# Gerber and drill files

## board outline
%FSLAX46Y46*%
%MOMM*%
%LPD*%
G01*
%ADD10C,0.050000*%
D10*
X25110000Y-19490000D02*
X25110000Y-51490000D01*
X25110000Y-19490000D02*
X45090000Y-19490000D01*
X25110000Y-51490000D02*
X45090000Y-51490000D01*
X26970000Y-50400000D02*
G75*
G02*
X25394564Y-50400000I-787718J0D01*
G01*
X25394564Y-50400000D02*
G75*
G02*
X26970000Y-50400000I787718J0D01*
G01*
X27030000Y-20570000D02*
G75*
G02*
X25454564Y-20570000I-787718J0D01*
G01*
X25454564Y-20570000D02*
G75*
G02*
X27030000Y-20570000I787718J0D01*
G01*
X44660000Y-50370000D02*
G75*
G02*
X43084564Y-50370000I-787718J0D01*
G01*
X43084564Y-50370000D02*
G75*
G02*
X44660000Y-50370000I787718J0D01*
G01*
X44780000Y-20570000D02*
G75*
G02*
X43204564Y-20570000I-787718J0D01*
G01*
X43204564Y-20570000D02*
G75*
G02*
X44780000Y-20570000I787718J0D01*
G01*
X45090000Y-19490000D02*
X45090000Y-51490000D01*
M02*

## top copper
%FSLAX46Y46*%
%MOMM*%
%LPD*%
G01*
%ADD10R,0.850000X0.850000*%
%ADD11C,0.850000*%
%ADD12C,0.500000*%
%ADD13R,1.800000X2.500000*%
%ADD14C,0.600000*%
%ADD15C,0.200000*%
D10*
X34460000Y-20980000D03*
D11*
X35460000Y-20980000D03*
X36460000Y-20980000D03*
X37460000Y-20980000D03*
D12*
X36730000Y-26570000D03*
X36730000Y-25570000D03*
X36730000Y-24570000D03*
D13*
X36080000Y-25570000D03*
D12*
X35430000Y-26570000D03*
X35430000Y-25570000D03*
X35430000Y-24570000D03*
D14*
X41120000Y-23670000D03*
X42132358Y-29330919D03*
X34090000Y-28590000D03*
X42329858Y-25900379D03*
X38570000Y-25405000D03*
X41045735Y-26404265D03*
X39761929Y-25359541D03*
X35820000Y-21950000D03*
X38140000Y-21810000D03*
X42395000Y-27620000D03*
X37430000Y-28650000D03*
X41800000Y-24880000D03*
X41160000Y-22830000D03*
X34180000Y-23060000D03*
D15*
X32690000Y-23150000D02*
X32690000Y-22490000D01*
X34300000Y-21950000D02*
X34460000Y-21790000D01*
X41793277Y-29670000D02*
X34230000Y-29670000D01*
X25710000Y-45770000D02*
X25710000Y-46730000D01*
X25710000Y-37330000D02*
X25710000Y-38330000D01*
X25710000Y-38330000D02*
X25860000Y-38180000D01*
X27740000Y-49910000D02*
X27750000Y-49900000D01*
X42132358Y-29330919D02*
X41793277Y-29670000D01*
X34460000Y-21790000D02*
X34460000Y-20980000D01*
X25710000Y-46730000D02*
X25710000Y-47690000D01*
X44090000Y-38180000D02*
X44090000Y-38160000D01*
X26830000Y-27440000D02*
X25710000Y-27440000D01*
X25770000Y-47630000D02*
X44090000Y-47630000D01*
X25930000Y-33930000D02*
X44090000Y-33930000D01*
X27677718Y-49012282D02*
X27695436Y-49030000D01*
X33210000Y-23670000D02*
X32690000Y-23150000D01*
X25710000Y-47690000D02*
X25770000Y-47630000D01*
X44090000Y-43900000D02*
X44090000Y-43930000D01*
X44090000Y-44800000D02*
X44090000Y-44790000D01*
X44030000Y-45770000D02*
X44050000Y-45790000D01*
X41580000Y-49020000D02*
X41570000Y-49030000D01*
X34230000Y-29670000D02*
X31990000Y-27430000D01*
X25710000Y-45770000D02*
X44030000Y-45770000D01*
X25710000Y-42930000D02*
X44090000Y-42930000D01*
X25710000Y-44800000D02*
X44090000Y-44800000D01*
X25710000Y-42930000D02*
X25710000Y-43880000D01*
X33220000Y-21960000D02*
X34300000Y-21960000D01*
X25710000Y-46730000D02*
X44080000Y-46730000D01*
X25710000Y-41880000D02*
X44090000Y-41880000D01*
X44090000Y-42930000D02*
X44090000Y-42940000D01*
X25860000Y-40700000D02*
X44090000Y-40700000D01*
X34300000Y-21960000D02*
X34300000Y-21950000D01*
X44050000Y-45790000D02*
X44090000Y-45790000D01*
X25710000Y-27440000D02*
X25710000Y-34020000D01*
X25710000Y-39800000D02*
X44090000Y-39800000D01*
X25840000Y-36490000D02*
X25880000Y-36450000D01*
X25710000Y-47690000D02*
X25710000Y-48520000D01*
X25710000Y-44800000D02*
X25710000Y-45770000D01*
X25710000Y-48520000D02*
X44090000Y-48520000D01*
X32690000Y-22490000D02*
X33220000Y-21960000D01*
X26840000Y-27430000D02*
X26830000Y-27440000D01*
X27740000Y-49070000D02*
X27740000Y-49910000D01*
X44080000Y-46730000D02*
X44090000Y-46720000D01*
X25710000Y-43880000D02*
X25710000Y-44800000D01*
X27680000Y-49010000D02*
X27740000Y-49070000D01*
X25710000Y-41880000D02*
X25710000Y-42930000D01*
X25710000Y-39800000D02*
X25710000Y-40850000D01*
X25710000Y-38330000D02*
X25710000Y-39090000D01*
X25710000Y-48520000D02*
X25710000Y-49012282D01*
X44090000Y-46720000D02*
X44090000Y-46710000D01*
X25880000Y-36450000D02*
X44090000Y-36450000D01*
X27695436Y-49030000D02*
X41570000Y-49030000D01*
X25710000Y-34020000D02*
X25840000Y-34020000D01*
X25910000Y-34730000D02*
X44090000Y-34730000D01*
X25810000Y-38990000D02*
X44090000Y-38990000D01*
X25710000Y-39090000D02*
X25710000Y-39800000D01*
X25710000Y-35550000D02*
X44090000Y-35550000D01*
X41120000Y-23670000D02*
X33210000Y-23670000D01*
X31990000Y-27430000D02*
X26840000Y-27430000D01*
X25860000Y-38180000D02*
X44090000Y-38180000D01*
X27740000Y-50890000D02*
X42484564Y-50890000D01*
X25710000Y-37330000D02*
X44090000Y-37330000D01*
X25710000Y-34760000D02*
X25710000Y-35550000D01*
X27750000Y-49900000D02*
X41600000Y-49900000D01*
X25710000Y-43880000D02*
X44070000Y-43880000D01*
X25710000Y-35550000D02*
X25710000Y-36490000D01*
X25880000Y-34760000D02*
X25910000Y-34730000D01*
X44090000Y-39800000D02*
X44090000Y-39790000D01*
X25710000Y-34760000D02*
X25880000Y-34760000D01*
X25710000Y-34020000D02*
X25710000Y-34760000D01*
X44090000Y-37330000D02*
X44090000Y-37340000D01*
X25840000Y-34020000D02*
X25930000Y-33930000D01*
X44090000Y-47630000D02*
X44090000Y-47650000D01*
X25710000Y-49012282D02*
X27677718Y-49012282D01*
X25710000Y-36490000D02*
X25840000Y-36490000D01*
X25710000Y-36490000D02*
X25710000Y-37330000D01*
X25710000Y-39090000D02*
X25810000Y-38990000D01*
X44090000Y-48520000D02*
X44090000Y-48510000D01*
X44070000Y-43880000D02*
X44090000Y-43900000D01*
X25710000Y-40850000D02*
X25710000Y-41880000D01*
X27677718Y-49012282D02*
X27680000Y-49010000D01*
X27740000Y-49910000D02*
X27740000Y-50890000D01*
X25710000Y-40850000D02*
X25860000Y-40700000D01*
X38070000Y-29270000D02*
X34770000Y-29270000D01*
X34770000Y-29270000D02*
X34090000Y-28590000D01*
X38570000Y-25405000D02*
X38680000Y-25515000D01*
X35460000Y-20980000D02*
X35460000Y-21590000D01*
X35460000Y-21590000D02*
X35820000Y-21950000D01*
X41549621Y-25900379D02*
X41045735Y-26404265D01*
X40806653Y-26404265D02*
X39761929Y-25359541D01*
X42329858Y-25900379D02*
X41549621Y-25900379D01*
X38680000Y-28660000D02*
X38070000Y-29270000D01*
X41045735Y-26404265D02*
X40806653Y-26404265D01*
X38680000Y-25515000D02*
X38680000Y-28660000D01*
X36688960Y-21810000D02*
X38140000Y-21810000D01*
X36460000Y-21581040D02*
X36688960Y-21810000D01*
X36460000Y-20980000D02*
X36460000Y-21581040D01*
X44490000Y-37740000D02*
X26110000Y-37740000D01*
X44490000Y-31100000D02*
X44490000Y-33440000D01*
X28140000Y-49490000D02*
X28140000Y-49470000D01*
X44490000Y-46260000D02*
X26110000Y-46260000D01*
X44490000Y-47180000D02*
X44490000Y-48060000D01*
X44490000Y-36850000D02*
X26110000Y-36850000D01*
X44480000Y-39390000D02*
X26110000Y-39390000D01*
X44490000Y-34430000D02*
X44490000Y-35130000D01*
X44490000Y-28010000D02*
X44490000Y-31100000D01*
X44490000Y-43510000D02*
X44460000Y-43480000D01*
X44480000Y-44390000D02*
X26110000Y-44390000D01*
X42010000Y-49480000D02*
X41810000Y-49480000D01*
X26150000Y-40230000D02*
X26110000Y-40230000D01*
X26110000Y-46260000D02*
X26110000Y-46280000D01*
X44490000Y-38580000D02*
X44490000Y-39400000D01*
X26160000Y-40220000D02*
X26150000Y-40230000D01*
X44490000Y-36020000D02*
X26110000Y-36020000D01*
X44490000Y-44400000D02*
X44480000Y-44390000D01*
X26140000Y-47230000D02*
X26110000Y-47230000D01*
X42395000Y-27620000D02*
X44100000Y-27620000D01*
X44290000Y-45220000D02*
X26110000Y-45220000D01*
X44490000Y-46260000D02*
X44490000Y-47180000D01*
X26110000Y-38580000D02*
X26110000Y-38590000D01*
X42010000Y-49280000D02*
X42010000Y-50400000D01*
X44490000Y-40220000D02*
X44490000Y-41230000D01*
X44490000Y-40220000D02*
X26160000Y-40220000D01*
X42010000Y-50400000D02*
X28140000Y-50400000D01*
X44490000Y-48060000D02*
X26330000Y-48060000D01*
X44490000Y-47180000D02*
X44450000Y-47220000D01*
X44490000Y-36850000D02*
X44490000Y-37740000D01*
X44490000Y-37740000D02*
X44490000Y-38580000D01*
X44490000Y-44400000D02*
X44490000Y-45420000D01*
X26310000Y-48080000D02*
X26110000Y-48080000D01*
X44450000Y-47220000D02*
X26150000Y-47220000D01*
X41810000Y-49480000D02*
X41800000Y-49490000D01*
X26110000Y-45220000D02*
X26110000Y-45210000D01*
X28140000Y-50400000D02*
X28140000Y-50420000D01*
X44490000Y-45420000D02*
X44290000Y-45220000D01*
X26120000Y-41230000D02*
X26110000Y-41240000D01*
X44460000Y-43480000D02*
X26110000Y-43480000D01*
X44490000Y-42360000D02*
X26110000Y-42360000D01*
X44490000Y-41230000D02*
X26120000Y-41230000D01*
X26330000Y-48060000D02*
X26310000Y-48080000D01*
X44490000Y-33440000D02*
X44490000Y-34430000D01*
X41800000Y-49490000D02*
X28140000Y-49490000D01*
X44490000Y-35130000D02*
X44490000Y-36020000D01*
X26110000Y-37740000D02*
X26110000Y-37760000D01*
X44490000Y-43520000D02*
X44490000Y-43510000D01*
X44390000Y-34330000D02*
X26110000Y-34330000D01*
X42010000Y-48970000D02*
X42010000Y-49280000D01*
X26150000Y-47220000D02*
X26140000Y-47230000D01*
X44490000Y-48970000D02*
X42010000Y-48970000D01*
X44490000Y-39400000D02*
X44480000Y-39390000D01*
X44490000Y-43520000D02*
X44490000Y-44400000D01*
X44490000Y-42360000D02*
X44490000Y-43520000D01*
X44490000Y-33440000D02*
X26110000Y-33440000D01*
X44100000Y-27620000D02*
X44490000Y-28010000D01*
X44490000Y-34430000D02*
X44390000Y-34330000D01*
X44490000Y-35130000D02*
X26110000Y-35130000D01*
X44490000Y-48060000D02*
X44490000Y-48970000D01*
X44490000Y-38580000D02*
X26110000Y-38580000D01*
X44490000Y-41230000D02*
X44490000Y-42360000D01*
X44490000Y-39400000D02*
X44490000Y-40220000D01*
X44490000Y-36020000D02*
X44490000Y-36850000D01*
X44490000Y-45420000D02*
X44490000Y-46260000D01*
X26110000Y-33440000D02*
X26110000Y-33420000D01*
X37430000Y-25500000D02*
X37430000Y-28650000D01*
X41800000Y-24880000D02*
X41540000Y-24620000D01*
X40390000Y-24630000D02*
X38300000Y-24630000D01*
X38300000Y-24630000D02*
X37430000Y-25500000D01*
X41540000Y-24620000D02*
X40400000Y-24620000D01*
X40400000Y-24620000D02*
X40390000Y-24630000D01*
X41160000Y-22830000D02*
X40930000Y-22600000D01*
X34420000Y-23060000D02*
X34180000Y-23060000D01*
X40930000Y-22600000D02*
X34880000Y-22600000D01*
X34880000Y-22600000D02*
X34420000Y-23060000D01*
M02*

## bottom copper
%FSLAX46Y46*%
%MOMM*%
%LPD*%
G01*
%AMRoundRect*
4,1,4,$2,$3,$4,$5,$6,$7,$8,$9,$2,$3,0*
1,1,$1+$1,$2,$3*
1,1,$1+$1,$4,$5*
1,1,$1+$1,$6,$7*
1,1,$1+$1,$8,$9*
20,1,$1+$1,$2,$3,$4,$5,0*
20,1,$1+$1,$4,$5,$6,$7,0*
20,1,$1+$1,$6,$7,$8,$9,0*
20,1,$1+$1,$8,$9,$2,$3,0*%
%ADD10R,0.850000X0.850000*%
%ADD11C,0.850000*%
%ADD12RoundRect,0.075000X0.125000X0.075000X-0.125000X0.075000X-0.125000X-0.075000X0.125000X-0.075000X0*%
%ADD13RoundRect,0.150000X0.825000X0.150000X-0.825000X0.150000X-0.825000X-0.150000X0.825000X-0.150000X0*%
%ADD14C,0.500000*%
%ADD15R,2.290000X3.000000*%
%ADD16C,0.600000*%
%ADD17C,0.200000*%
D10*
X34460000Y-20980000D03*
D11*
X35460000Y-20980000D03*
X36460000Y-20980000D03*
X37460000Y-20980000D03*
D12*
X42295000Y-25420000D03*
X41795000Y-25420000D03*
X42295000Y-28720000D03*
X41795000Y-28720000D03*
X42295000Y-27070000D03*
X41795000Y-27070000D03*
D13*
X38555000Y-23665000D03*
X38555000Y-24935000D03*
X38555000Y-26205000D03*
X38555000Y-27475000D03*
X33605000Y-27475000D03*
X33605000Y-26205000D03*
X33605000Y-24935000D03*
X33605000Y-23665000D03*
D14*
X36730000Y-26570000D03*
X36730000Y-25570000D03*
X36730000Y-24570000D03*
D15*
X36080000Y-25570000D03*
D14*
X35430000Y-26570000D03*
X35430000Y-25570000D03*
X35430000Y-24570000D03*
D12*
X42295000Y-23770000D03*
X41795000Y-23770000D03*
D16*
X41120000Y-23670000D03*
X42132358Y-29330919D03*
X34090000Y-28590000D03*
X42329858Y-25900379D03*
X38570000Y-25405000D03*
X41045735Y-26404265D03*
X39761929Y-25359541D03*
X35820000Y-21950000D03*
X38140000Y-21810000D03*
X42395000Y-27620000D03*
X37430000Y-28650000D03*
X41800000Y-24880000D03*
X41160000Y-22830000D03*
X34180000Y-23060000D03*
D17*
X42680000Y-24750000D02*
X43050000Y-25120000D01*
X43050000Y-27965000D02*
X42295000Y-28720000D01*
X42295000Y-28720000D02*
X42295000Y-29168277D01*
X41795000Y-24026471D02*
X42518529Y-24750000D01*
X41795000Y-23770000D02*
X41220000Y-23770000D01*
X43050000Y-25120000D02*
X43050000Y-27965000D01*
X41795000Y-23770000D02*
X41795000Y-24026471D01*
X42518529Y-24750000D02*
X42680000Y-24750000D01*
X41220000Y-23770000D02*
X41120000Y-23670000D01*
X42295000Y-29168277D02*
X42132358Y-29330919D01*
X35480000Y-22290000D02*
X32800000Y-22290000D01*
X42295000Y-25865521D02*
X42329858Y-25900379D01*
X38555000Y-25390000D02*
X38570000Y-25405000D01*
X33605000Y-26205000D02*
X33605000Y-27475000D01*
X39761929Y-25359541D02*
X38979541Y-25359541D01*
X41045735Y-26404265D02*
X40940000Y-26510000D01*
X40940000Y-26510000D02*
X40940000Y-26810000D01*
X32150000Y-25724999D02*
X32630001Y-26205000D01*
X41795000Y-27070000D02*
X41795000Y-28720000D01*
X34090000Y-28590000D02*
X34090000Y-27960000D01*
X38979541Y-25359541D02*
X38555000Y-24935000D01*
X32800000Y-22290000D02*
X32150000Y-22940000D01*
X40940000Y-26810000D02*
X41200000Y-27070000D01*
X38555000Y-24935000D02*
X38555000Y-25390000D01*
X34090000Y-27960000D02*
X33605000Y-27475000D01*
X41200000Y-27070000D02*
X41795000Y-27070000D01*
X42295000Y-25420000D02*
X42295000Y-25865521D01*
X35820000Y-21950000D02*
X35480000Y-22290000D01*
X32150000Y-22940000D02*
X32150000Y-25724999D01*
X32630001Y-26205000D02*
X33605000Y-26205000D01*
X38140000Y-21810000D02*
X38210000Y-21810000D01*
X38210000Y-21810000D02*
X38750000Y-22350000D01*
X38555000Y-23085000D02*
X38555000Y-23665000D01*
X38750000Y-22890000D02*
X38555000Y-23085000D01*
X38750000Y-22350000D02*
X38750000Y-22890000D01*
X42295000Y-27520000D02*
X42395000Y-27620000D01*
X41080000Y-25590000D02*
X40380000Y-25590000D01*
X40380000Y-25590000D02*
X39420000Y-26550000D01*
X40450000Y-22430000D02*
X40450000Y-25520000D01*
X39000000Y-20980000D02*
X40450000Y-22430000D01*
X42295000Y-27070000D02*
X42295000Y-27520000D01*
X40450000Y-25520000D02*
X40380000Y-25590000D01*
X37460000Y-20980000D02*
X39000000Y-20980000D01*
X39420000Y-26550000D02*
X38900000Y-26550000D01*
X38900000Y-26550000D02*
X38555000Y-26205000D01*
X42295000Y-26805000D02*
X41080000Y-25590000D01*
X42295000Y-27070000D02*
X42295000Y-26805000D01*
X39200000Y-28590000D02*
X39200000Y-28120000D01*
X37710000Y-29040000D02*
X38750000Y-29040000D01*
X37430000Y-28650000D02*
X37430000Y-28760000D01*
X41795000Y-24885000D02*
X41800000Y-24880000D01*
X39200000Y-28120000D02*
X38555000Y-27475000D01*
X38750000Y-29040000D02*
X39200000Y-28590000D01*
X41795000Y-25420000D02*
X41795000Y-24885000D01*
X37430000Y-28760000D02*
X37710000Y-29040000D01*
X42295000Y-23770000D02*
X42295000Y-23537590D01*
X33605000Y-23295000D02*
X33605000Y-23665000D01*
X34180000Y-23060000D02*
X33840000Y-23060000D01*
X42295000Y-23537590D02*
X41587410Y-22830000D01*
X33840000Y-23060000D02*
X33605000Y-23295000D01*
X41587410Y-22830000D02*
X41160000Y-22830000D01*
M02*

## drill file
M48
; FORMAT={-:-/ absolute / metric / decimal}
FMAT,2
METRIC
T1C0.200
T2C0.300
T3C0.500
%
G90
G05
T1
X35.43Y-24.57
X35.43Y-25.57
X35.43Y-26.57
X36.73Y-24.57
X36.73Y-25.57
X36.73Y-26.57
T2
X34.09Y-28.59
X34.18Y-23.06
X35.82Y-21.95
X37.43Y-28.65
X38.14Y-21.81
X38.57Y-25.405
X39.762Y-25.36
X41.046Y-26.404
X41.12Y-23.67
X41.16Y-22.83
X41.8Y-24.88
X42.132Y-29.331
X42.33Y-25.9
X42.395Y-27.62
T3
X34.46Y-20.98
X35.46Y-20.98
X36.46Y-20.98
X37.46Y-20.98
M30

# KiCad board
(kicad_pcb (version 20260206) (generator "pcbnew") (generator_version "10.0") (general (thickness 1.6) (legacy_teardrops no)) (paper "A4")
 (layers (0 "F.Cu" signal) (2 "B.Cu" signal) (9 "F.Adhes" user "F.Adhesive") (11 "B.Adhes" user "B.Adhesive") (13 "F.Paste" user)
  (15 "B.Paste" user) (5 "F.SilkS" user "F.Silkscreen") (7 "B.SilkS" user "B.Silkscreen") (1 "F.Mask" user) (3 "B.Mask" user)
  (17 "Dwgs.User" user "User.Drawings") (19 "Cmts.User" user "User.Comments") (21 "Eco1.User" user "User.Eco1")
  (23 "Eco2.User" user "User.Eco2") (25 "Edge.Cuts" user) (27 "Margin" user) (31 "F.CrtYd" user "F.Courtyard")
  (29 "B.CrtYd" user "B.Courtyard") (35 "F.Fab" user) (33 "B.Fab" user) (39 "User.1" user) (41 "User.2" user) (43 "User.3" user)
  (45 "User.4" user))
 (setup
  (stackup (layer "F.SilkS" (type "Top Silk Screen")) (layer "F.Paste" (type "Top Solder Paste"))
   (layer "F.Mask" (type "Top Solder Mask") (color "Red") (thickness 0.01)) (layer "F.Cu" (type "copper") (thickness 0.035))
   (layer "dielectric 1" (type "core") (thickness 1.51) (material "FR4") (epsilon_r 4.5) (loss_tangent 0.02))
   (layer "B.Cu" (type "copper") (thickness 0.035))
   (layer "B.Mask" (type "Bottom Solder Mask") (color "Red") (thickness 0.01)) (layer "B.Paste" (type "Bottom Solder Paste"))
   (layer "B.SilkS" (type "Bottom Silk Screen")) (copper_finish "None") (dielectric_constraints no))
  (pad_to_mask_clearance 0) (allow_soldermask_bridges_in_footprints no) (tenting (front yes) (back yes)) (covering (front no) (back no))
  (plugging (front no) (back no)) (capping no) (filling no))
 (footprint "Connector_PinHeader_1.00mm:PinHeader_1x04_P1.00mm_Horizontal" (layer "F.Cu") (at 34.46 20.98 90)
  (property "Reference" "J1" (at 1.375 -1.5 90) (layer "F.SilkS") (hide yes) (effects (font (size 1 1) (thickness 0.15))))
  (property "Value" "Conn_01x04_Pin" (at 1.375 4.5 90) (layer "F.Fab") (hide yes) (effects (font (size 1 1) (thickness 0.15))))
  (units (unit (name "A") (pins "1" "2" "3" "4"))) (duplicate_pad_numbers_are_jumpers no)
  (pad "1" thru_hole rect (at 0 0 90) (size 0.85 0.85) (drill 0.5) (layers "*.Cu" "*.Mask") (remove_unused_layers no) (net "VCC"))
  (pad "2" thru_hole circle (at 0 1 90) (size 0.85 0.85) (drill 0.5) (layers "*.Cu" "*.Mask") (remove_unused_layers no) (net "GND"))
  (pad "3" thru_hole circle (at 0 2 90) (size 0.85 0.85) (drill 0.5) (layers "*.Cu" "*.Mask") (remove_unused_layers no) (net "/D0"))
  (pad "4" thru_hole circle (at 0 3 90) (size 0.85 0.85) (drill 0.5) (layers "*.Cu" "*.Mask") (remove_unused_layers no) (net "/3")))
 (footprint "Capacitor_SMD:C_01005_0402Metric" (layer "B.Cu") (at 42.045 25.42 180)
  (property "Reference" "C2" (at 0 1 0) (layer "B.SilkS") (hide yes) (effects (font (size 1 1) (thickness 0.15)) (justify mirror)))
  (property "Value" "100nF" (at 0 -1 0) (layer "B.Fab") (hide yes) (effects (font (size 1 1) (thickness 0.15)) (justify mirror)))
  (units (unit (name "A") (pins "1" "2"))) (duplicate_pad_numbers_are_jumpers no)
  (pad "" smd roundrect (at -0.275 0 180) (size 0.27 0.27) (layers "B.Paste") (roundrect_rratio 0.25))
  (pad "" smd roundrect (at 0.275 0 180) (size 0.27 0.27) (layers "B.Paste") (roundrect_rratio 0.25))
  (pad "1" smd roundrect (at -0.25 0 180) (size 0.4 0.3) (layers "B.Cu" "B.Mask") (roundrect_rratio 0.25) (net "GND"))
  (pad "2" smd roundrect (at 0.25 0 180) (size 0.4 0.3) (layers "B.Cu" "B.Mask") (roundrect_rratio 0.25) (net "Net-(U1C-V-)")))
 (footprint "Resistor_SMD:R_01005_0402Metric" (layer "B.Cu") (at 42.045 28.72 180)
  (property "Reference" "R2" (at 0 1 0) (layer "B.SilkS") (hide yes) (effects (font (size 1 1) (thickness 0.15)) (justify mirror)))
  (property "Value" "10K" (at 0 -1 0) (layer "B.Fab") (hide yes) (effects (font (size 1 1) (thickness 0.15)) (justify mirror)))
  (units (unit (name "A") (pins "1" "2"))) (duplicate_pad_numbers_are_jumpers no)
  (pad "" smd roundrect (at -0.275 0 180) (size 0.27 0.27) (layers "B.Paste") (roundrect_rratio 0.25))
  (pad "" smd roundrect (at 0.275 0 180) (size 0.27 0.27) (layers "B.Paste") (roundrect_rratio 0.25))
  (pad "1" smd roundrect (at -0.25 0 180) (size 0.4 0.3) (layers "B.Cu" "B.Mask") (roundrect_rratio 0.25) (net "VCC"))
  (pad "2" smd roundrect (at 0.25 0 180) (size 0.4 0.3) (layers "B.Cu" "B.Mask") (roundrect_rratio 0.25) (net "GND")))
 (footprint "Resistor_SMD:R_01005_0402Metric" (layer "B.Cu") (at 42.045 27.07 180)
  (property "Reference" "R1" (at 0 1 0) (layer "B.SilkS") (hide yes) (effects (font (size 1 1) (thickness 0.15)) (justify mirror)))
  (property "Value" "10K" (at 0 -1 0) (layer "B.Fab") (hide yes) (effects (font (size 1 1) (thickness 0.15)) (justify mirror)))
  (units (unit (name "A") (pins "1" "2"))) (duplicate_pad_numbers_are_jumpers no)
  (pad "" smd roundrect (at -0.275 0 180) (size 0.27 0.27) (layers "B.Paste") (roundrect_rratio 0.25))
  (pad "" smd roundrect (at 0.275 0 180) (size 0.27 0.27) (layers "B.Paste") (roundrect_rratio 0.25))
  (pad "1" smd roundrect (at -0.25 0 180) (size 0.4 0.3) (layers "B.Cu" "B.Mask") (roundrect_rratio 0.25) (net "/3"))
  (pad "2" smd roundrect (at 0.25 0 180) (size 0.4 0.3) (layers "B.Cu" "B.Mask") (roundrect_rratio 0.25) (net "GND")))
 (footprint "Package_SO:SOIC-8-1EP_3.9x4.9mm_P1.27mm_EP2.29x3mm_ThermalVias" (layer "B.Cu") (at 36.08 25.57 180)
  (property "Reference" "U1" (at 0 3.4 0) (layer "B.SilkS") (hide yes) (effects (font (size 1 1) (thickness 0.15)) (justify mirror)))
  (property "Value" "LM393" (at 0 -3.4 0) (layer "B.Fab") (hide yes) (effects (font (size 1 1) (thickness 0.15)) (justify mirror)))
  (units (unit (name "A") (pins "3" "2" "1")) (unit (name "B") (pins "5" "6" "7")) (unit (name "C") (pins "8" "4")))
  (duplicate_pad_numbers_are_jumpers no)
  (pad "" smd roundrect (at -0.57 -0.75 180) (size 0.96 1.25) (layers "B.Paste") (roundrect_rratio 0.25))
  (pad "" smd roundrect (at -0.57 0.75 180) (size 0.96 1.25) (layers "B.Paste") (roundrect_rratio 0.25))
  (pad "" smd roundrect (at 0.57 -0.75 180) (size 0.96 1.25) (layers "B.Paste") (roundrect_rratio 0.25))
  (pad "" smd roundrect (at 0.57 0.75 180) (size 0.96 1.25) (layers "B.Paste") (roundrect_rratio 0.25))
  (pad "1" smd roundrect (at -2.475 1.905 180) (size 1.95 0.6) (layers "B.Cu" "B.Mask" "B.Paste") (roundrect_rratio 0.25) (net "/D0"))
  (pad "2" smd roundrect (at -2.475 0.635 180) (size 1.95 0.6) (layers "B.Cu" "B.Mask" "B.Paste") (roundrect_rratio 0.25) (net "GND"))
  (pad "3" smd roundrect (at -2.475 -0.635 180) (size 1.95 0.6) (layers "B.Cu" "B.Mask" "B.Paste") (roundrect_rratio 0.25) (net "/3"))
  (pad "4" smd roundrect (at -2.475 -1.905 180) (size 1.95 0.6) (layers "B.Cu" "B.Mask" "B.Paste") (roundrect_rratio 0.25)
   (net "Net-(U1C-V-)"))
  (pad "5" smd roundrect (at 2.475 -1.905 180) (size 1.95 0.6) (layers "B.Cu" "B.Mask" "B.Paste") (roundrect_rratio 0.25) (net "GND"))
  (pad "6" smd roundrect (at 2.475 -0.635 180) (size 1.95 0.6) (layers "B.Cu" "B.Mask" "B.Paste") (roundrect_rratio 0.25) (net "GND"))
  (pad "7" smd roundrect (at 2.475 0.635 180) (size 1.95 0.6) (layers "B.Cu" "B.Mask" "B.Paste") (roundrect_rratio 0.25)
   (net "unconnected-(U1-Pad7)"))
  (pad "8" smd roundrect (at 2.475 1.905 180) (size 1.95 0.6) (layers "B.Cu" "B.Mask" "B.Paste") (roundrect_rratio 0.25)
   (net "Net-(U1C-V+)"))
  (pad "9" thru_hole circle (at -0.65 -1 180) (size 0.5 0.5) (drill 0.2) (layers "*.Cu") (remove_unused_layers no))
  (pad "9" thru_hole circle (at -0.65 0 180) (size 0.5 0.5) (drill 0.2) (layers "*.Cu") (remove_unused_layers no))
  (pad "9" thru_hole circle (at -0.65 1 180) (size 0.5 0.5) (drill 0.2) (layers "*.Cu") (remove_unused_layers no))
  (pad "9" smd rect (at 0 0 180) (size 1.8 2.5) (layers "F.Cu") (zone_connect 2))
  (pad "9" smd rect (at 0 0 180) (size 2.29 3) (layers "B.Cu" "B.Mask") (zone_connect 2))
  (pad "9" thru_hole circle (at 0.65 -1 180) (size 0.5 0.5) (drill 0.2) (layers "*.Cu") (remove_unused_layers no))
  (pad "9" thru_hole circle (at 0.65 0 180) (size 0.5 0.5) (drill 0.2) (layers "*.Cu") (remove_unused_layers no))
  (pad "9" thru_hole circle (at 0.65 1 180) (size 0.5 0.5) (drill 0.2) (layers "*.Cu") (remove_unused_layers no)))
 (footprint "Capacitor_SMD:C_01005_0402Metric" (layer "B.Cu") (at 42.045 23.77 180)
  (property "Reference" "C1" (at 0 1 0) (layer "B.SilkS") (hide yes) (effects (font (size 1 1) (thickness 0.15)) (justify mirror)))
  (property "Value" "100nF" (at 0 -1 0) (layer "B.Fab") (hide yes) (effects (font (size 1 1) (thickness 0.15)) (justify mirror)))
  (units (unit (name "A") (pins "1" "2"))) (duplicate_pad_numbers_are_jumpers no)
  (pad "" smd roundrect (at -0.275 0 180) (size 0.27 0.27) (layers "B.Paste") (roundrect_rratio 0.25))
  (pad "" smd roundrect (at 0.275 0 180) (size 0.27 0.27) (layers "B.Paste") (roundrect_rratio 0.25))
  (pad "1" smd roundrect (at -0.25 0 180) (size 0.4 0.3) (layers "B.Cu" "B.Mask") (roundrect_rratio 0.25) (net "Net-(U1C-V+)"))
  (pad "2" smd roundrect (at 0.25 0 180) (size 0.4 0.3) (layers "B.Cu" "B.Mask") (roundrect_rratio 0.25) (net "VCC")))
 (gr_line (start 25.11 19.49) (end 25.11 51.49) (stroke (width 0.05) (type default)) (layer "Edge.Cuts"))
 (gr_line (start 25.11 19.49) (end 45.09 19.49) (stroke (width 0.05) (type default)) (layer "Edge.Cuts"))
 (gr_line (start 25.11 51.49) (end 45.09 51.49) (stroke (width 0.05) (type default)) (layer "Edge.Cuts"))
 (gr_circle (center 26.182282 50.4) (end 25.752282 49.74) (stroke (width 0.05) (type default)) (fill no) (layer "Edge.Cuts"))
 (gr_circle (center 26.242282 20.57) (end 25.812282 19.91) (stroke (width 0.05) (type default)) (fill no) (layer "Edge.Cuts"))
 (gr_circle (center 43.872282 50.37) (end 43.442282 49.71) (stroke (width 0.05) (type default)) (fill no) (layer "Edge.Cuts"))
 (gr_circle (center 43.992282 20.57) (end 43.562282 19.91) (stroke (width 0.05) (type default)) (fill no) (layer "Edge.Cuts"))
 (gr_line (start 45.09 19.49) (end 45.09 51.49) (stroke (width 0.05) (type default)) (layer "Edge.Cuts"))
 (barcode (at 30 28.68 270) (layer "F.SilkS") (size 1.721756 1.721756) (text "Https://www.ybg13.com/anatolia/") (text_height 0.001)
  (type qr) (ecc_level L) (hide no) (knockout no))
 (segment (start 32.69 23.15) (end 32.69 22.49) (width 0.2) (layer "F.Cu") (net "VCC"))
 (segment (start 34.3 21.95) (end 34.46 21.79) (width 0.2) (layer "F.Cu") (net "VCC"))
 (segment (start 41.793277 29.67) (end 34.23 29.67) (width 0.2) (layer "F.Cu") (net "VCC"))
 (segment (start 25.71 45.77) (end 25.71 46.73) (width 0.2) (layer "F.Cu") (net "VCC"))
 (segment (start 25.71 37.33) (end 25.71 38.33) (width 0.2) (layer "F.Cu") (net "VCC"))
 (segment (start 25.71 38.33) (end 25.86 38.18) (width 0.2) (layer "F.Cu") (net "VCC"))
 (segment (start 27.74 49.91) (end 27.75 49.9) (width 0.2) (layer "F.Cu") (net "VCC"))
 (segment (start 42.132358 29.330919) (end 41.793277 29.67) (width 0.2) (layer "F.Cu") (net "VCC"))
 (segment (start 34.46 21.79) (end 34.46 20.98) (width 0.2) (layer "F.Cu") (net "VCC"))
 (segment (start 25.71 46.73) (end 25.71 47.69) (width 0.2) (layer "F.Cu") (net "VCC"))
 (segment (start 44.09 38.18) (end 44.09 38.16) (width 0.2) (layer "F.Cu") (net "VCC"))
 (segment (start 26.83 27.44) (end 25.71 27.44) (width 0.2) (layer "F.Cu") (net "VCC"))
 (segment (start 25.77 47.63) (end 44.09 47.63) (width 0.2) (layer "F.Cu") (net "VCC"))
 (segment (start 25.93 33.93) (end 44.09 33.93) (width 0.2) (layer "F.Cu") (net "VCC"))
 (segment (start 27.677718 49.012282) (end 27.695436 49.03) (width 0.2) (layer "F.Cu") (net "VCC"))
 (segment (start 33.21 23.67) (end 32.69 23.15) (width 0.2) (layer "F.Cu") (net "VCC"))
 (segment (start 25.71 47.69) (end 25.77 47.63) (width 0.2) (layer "F.Cu") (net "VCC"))
 (segment (start 44.09 43.9) (end 44.09 43.93) (width 0.2) (layer "F.Cu") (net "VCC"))
 (segment (start 44.09 44.8) (end 44.09 44.79) (width 0.2) (layer "F.Cu") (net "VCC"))
 (segment (start 44.03 45.77) (end 44.05 45.79) (width 0.2) (layer "F.Cu") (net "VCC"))
 (segment (start 41.58 49.02) (end 41.57 49.03) (width 0.2) (layer "F.Cu") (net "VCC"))
 (segment (start 34.23 29.67) (end 31.99 27.43) (width 0.2) (layer "F.Cu") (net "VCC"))
 (segment (start 25.71 45.77) (end 44.03 45.77) (width 0.2) (layer "F.Cu") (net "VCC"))
 (segment (start 25.71 42.93) (end 44.09 42.93) (width 0.2) (layer "F.Cu") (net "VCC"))
 (segment (start 25.71 44.8) (end 44.09 44.8) (width 0.2) (layer "F.Cu") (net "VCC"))
 (segment (start 25.71 42.93) (end 25.71 43.88) (width 0.2) (layer "F.Cu") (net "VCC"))
 (segment (start 33.22 21.96) (end 34.3 21.96) (width 0.2) (layer "F.Cu") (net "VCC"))
 (segment (start 25.71 46.73) (end 44.08 46.73) (width 0.2) (layer "F.Cu") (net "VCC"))
 (segment (start 25.71 41.88) (end 44.09 41.88) (width 0.2) (layer "F.Cu") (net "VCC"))
 (segment (start 44.09 42.93) (end 44.09 42.94) (width 0.2) (layer "F.Cu") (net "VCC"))
 (segment (start 25.86 40.7) (end 44.09 40.7) (width 0.2) (layer "F.Cu") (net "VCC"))
 (segment (start 34.3 21.96) (end 34.3 21.95) (width 0.2) (layer "F.Cu") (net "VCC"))
 (segment (start 44.05 45.79) (end 44.09 45.79) (width 0.2) (layer "F.Cu") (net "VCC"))
 (segment (start 25.71 27.44) (end 25.71 34.02) (width 0.2) (layer "F.Cu") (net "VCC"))
 (segment (start 25.71 39.8) (end 44.09 39.8) (width 0.2) (layer "F.Cu") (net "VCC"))
 (segment (start 25.84 36.49) (end 25.88 36.45) (width 0.2) (layer "F.Cu") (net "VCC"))
 (segment (start 25.71 47.69) (end 25.71 48.52) (width 0.2) (layer "F.Cu") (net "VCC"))
 (segment (start 25.71 44.8) (end 25.71 45.77) (width 0.2) (layer "F.Cu") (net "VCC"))
 (segment (start 25.71 48.52) (end 44.09 48.52) (width 0.2) (layer "F.Cu") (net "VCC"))
 (segment (start 32.69 22.49) (end 33.22 21.96) (width 0.2) (layer "F.Cu") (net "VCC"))
 (segment (start 26.84 27.43) (end 26.83 27.44) (width 0.2) (layer "F.Cu") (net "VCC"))
 (segment (start 27.74 49.07) (end 27.74 49.91) (width 0.2) (layer "F.Cu") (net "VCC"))
 (segment (start 44.08 46.73) (end 44.09 46.72) (width 0.2) (layer "F.Cu") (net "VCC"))
 (segment (start 25.71 43.88) (end 25.71 44.8) (width 0.2) (layer "F.Cu") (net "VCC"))
 (segment (start 27.68 49.01) (end 27.74 49.07) (width 0.2) (layer "F.Cu") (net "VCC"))
 (segment (start 25.71 41.88) (end 25.71 42.93) (width 0.2) (layer "F.Cu") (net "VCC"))
 (segment (start 25.71 39.8) (end 25.71 40.85) (width 0.2) (layer "F.Cu") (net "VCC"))
 (segment (start 25.71 38.33) (end 25.71 39.09) (width 0.2) (layer "F.Cu") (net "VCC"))
 (segment (start 25.71 48.52) (end 25.71 49.012282) (width 0.2) (layer "F.Cu") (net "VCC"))
 (segment (start 44.09 46.72) (end 44.09 46.71) (width 0.2) (layer "F.Cu") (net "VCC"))
 (segment (start 25.88 36.45) (end 44.09 36.45) (width 0.2) (layer "F.Cu") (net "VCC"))
 (segment (start 27.695436 49.03) (end 41.57 49.03) (width 0.2) (layer "F.Cu") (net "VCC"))
 (segment (start 25.71 34.02) (end 25.84 34.02) (width 0.2) (layer "F.Cu") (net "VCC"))
 (segment (start 25.91 34.73) (end 44.09 34.73) (width 0.2) (layer "F.Cu") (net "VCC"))
 (segment (start 25.81 38.99) (end 44.09 38.99) (width 0.2) (layer "F.Cu") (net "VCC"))
 (segment (start 25.71 39.09) (end 25.71 39.8) (width 0.2) (layer "F.Cu") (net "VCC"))
 (segment (start 25.71 35.55) (end 44.09 35.55) (width 0.2) (layer "F.Cu") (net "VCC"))
 (segment (start 41.12 23.67) (end 33.21 23.67) (width 0.2) (layer "F.Cu") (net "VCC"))
 (segment (start 31.99 27.43) (end 26.84 27.43) (width 0.2) (layer "F.Cu") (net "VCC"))
 (segment (start 25.86 38.18) (end 44.09 38.18) (width 0.2) (layer "F.Cu") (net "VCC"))
 (segment (start 27.74 50.89) (end 42.484564 50.89) (width 0.2) (layer "F.Cu") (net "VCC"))
 (segment (start 25.71 37.33) (end 44.09 37.33) (width 0.2) (layer "F.Cu") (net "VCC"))
 (segment (start 25.71 34.76) (end 25.71 35.55) (width 0.2) (layer "F.Cu") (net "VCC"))
 (segment (start 27.75 49.9) (end 41.6 49.9) (width 0.2) (layer "F.Cu") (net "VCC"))
 (segment (start 25.71 43.88) (end 44.07 43.88) (width 0.2) (layer "F.Cu") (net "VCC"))
 (segment (start 25.71 35.55) (end 25.71 36.49) (width 0.2) (layer "F.Cu") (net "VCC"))
 (segment (start 25.88 34.76) (end 25.91 34.73) (width 0.2) (layer "F.Cu") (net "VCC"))
 (segment (start 44.09 39.8) (end 44.09 39.79) (width 0.2) (layer "F.Cu") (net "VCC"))
 (segment (start 25.71 34.76) (end 25.88 34.76) (width 0.2) (layer "F.Cu") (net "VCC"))
 (segment (start 25.71 34.02) (end 25.71 34.76) (width 0.2) (layer "F.Cu") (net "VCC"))
 (segment (start 44.09 37.33) (end 44.09 37.34) (width 0.2) (layer "F.Cu") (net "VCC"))
 (segment (start 25.84 34.02) (end 25.93 33.93) (width 0.2) (layer "F.Cu") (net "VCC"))
 (segment (start 44.09 47.63) (end 44.09 47.65) (width 0.2) (layer "F.Cu") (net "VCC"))
 (segment (start 25.71 49.012282) (end 27.677718 49.012282) (width 0.2) (layer "F.Cu") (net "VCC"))
 (segment (start 25.71 36.49) (end 25.84 36.49) (width 0.2) (layer "F.Cu") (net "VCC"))
 (segment (start 25.71 36.49) (end 25.71 37.33) (width 0.2) (layer "F.Cu") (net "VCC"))
 (segment (start 25.71 39.09) (end 25.81 38.99) (width 0.2) (layer "F.Cu") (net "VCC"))
 (segment (start 44.09 48.52) (end 44.09 48.51) (width 0.2) (layer "F.Cu") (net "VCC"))
 (segment (start 44.07 43.88) (end 44.09 43.9) (width 0.2) (layer "F.Cu") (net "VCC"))
 (segment (start 25.71 40.85) (end 25.71 41.88) (width 0.2) (layer "F.Cu") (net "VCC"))
 (segment (start 27.677718 49.012282) (end 27.68 49.01) (width 0.2) (layer "F.Cu") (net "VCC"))
 (segment (start 27.74 49.91) (end 27.74 50.89) (width 0.2) (layer "F.Cu") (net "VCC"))
 (segment (start 25.71 40.85) (end 25.86 40.7) (width 0.2) (layer "F.Cu") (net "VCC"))
 (via (at 41.12 23.67) (size 0.6) (drill 0.3) (layers "F.Cu" "B.Cu") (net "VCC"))
 (via (at 42.132358 29.330919) (size 0.6) (drill 0.3) (layers "F.Cu" "B.Cu") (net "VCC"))
 (segment (start 42.68 24.75) (end 43.05 25.12) (width 0.2) (layer "B.Cu") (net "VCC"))
 (segment (start 43.05 27.965) (end 42.295 28.72) (width 0.2) (layer "B.Cu") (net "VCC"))
 (segment (start 42.295 28.72) (end 42.295 29.168277) (width 0.2) (layer "B.Cu") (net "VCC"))
 (segment (start 41.795 24.026471) (end 42.518529 24.75) (width 0.2) (layer "B.Cu") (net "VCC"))
 (segment (start 41.795 23.77) (end 41.22 23.77) (width 0.2) (layer "B.Cu") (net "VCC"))
 (segment (start 43.05 25.12) (end 43.05 27.965) (width 0.2) (layer "B.Cu") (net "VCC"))
 (segment (start 41.795 23.77) (end 41.795 24.026471) (width 0.2) (layer "B.Cu") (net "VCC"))
 (segment (start 42.518529 24.75) (end 42.68 24.75) (width 0.2) (layer "B.Cu") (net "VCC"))
 (segment (start 41.22 23.77) (end 41.12 23.67) (width 0.2) (layer "B.Cu") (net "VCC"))
 (segment (start 42.295 29.168277) (end 42.132358 29.330919) (width 0.2) (layer "B.Cu") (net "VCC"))
 (segment (start 38.07 29.27) (end 34.77 29.27) (width 0.2) (layer "F.Cu") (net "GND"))
 (segment (start 34.77 29.27) (end 34.09 28.59) (width 0.2) (layer "F.Cu") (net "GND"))
 (segment (start 38.57 25.405) (end 38.68 25.515) (width 0.2) (layer "F.Cu") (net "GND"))
 (segment (start 35.46 20.98) (end 35.46 21.59) (width 0.2) (layer "F.Cu") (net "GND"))
 (segment (start 35.46 21.59) (end 35.82 21.95) (width 0.2) (layer "F.Cu") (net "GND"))
 (segment (start 41.549621 25.900379) (end 41.045735 26.404265) (width 0.2) (layer "F.Cu") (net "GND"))
 (segment (start 40.806653 26.404265) (end 39.761929 25.359541) (width 0.2) (layer "F.Cu") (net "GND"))
 (segment (start 42.329858 25.900379) (end 41.549621 25.900379) (width 0.2) (layer "F.Cu") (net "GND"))
 (segment (start 38.68 28.66) (end 38.07 29.27) (width 0.2) (layer "F.Cu") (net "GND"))
 (segment (start 41.045735 26.404265) (end 40.806653 26.404265) (width 0.2) (layer "F.Cu") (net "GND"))
 (segment (start 38.68 25.515) (end 38.68 28.66) (width 0.2) (layer "F.Cu") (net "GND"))
 (via (at 34.09 28.59) (size 0.6) (drill 0.3) (layers "F.Cu" "B.Cu") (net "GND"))
 (via (at 42.329858 25.900379) (size 0.6) (drill 0.3) (layers "F.Cu" "B.Cu") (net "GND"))
 (via (at 38.57 25.405) (size 0.6) (drill 0.3) (layers "F.Cu" "B.Cu") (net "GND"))
 (via (at 41.045735 26.404265) (size 0.6) (drill 0.3) (layers "F.Cu" "B.Cu") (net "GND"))
 (via (at 39.761929 25.359541) (size 0.6) (drill 0.3) (layers "F.Cu" "B.Cu") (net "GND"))
 (via (at 35.82 21.95) (size 0.6) (drill 0.3) (layers "F.Cu" "B.Cu") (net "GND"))
 (segment (start 35.48 22.29) (end 32.8 22.29) (width 0.2) (layer "B.Cu") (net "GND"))
 (segment (start 42.295 25.865521) (end 42.329858 25.900379) (width 0.2) (layer "B.Cu") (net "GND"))
 (segment (start 38.555 25.39) (end 38.57 25.405) (width 0.2) (layer "B.Cu") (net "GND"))
 (segment (start 33.605 26.205) (end 33.605 27.475) (width 0.2) (layer "B.Cu") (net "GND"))
 (segment (start 39.761929 25.359541) (end 38.979541 25.359541) (width 0.2) (layer "B.Cu") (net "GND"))
 (segment (start 41.045735 26.404265) (end 40.94 26.51) (width 0.2) (layer "B.Cu") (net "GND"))
 (segment (start 40.94 26.51) (end 40.94 26.81) (width 0.2) (layer "B.Cu") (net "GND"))
 (segment (start 32.15 25.724999) (end 32.630001 26.205) (width 0.2) (layer "B.Cu") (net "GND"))
 (segment (start 41.795 27.07) (end 41.795 28.72) (width 0.2) (layer "B.Cu") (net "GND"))
 (segment (start 34.09 28.59) (end 34.09 27.96) (width 0.2) (layer "B.Cu") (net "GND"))
 (segment (start 38.979541 25.359541) (end 38.555 24.935) (width 0.2) (layer "B.Cu") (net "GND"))
 (segment (start 32.8 22.29) (end 32.15 22.94) (width 0.2) (layer "B.Cu") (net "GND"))
 (segment (start 40.94 26.81) (end 41.2 27.07) (width 0.2) (layer "B.Cu") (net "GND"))
 (segment (start 38.555 24.935) (end 38.555 25.39) (width 0.2) (layer "B.Cu") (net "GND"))
 (segment (start 34.09 27.96) (end 33.605 27.475) (width 0.2) (layer "B.Cu") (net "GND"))
 (segment (start 41.2 27.07) (end 41.795 27.07) (width 0.2) (layer "B.Cu") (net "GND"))
 (segment (start 42.295 25.42) (end 42.295 25.865521) (width 0.2) (layer "B.Cu") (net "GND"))
 (segment (start 35.82 21.95) (end 35.48 22.29) (width 0.2) (layer "B.Cu") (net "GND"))
 (segment (start 32.15 22.94) (end 32.15 25.724999) (width 0.2) (layer "B.Cu") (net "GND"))
 (segment (start 32.630001 26.205) (end 33.605 26.205) (width 0.2) (layer "B.Cu") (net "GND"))
 (segment (start 36.68896 21.81) (end 38.14 21.81) (width 0.2) (layer "F.Cu") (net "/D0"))
 (segment (start 36.46 21.58104) (end 36.68896 21.81) (width 0.2) (layer "F.Cu") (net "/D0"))
 (segment (start 36.46 20.98) (end 36.46 21.58104) (width 0.2) (layer "F.Cu") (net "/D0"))
 (via (at 38.14 21.81) (size 0.6) (drill 0.3) (layers "F.Cu" "B.Cu") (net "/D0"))
 (segment (start 38.14 21.81) (end 38.21 21.81) (width 0.2) (layer "B.Cu") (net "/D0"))
 (segment (start 38.21 21.81) (end 38.75 22.35) (width 0.2) (layer "B.Cu") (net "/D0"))
 (segment (start 38.555 23.085) (end 38.555 23.665) (width 0.2) (layer "B.Cu") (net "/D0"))
 (segment (start 38.75 22.89) (end 38.555 23.085) (width 0.2) (layer "B.Cu") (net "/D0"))
 (segment (start 38.75 22.35) (end 38.75 22.89) (width 0.2) (layer "B.Cu") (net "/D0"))
 (segment (start 44.49 37.74) (end 26.11 37.74) (width 0.2) (layer "F.Cu") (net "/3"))
 (segment (start 44.49 31.1) (end 44.49 33.44) (width 0.2) (layer "F.Cu") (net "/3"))
 (segment (start 28.14 49.49) (end 28.14 49.47) (width 0.2) (layer "F.Cu") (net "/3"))
 (segment (start 44.49 46.26) (end 26.11 46.26) (width 0.2) (layer "F.Cu") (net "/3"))
 (segment (start 44.49 47.18) (end 44.49 48.06) (width 0.2) (layer "F.Cu") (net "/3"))
 (segment (start 44.49 36.85) (end 26.11 36.85) (width 0.2) (layer "F.Cu") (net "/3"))
 (segment (start 44.48 39.39) (end 26.11 39.39) (width 0.2) (layer "F.Cu") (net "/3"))
 (segment (start 44.49 34.43) (end 44.49 35.13) (width 0.2) (layer "F.Cu") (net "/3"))
 (segment (start 44.49 28.01) (end 44.49 31.1) (width 0.2) (layer "F.Cu") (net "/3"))
 (segment (start 44.49 43.51) (end 44.46 43.48) (width 0.2) (layer "F.Cu") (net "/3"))
 (segment (start 44.48 44.39) (end 26.11 44.39) (width 0.2) (layer "F.Cu") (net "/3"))
 (segment (start 42.01 49.48) (end 41.81 49.48) (width 0.2) (layer "F.Cu") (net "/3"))
 (segment (start 26.15 40.23) (end 26.11 40.23) (width 0.2) (layer "F.Cu") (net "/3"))
 (segment (start 26.11 46.26) (end 26.11 46.28) (width 0.2) (layer "F.Cu") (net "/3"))
 (segment (start 44.49 38.58) (end 44.49 39.4) (width 0.2) (layer "F.Cu") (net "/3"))
 (segment (start 26.16 40.22) (end 26.15 40.23) (width 0.2) (layer "F.Cu") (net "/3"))
 (segment (start 44.49 36.02) (end 26.11 36.02) (width 0.2) (layer "F.Cu") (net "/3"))
 (segment (start 44.49 44.4) (end 44.48 44.39) (width 0.2) (layer "F.Cu") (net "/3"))
 (segment (start 26.14 47.23) (end 26.11 47.23) (width 0.2) (layer "F.Cu") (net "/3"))
 (segment (start 42.395 27.62) (end 44.1 27.62) (width 0.2) (layer "F.Cu") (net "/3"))
 (segment (start 44.29 45.22) (end 26.11 45.22) (width 0.2) (layer "F.Cu") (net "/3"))
 (segment (start 44.49 46.26) (end 44.49 47.18) (width 0.2) (layer "F.Cu") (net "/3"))
 (segment (start 26.11 38.58) (end 26.11 38.59) (width 0.2) (layer "F.Cu") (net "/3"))
 (segment (start 42.01 49.28) (end 42.01 50.4) (width 0.2) (layer "F.Cu") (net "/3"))
 (segment (start 44.49 40.22) (end 44.49 41.23) (width 0.2) (layer "F.Cu") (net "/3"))
 (segment (start 44.49 40.22) (end 26.16 40.22) (width 0.2) (layer "F.Cu") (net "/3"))
 (segment (start 42.01 50.4) (end 28.14 50.4) (width 0.2) (layer "F.Cu") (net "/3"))
 (segment (start 44.49 48.06) (end 26.33 48.06) (width 0.2) (layer "F.Cu") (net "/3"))
 (segment (start 44.49 47.18) (end 44.45 47.22) (width 0.2) (layer "F.Cu") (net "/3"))
 (segment (start 44.49 36.85) (end 44.49 37.74) (width 0.2) (layer "F.Cu") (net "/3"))
 (segment (start 44.49 37.74) (end 44.49 38.58) (width 0.2) (layer "F.Cu") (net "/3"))
 (segment (start 44.49 44.4) (end 44.49 45.42) (width 0.2) (layer "F.Cu") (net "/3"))
 (segment (start 26.31 48.08) (end 26.11 48.08) (width 0.2) (layer "F.Cu") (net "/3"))
 (segment (start 44.45 47.22) (end 26.15 47.22) (width 0.2) (layer "F.Cu") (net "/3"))
 (segment (start 41.81 49.48) (end 41.8 49.49) (width 0.2) (layer "F.Cu") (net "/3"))
 (segment (start 26.11 45.22) (end 26.11 45.21) (width 0.2) (layer "F.Cu") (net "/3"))
 (segment (start 28.14 50.4) (end 28.14 50.42) (width 0.2) (layer "F.Cu") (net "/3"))
 (segment (start 44.49 45.42) (end 44.29 45.22) (width 0.2) (layer "F.Cu") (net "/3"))
 (segment (start 26.12 41.23) (end 26.11 41.24) (width 0.2) (layer "F.Cu") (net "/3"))
 (segment (start 44.46 43.48) (end 26.11 43.48) (width 0.2) (layer "F.Cu") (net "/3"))
 (segment (start 44.49 42.36) (end 26.11 42.36) (width 0.2) (layer "F.Cu") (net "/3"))
 (segment (start 44.49 41.23) (end 26.12 41.23) (width 0.2) (layer "F.Cu") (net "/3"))
 (segment (start 26.33 48.06) (end 26.31 48.08) (width 0.2) (layer "F.Cu") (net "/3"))
 (segment (start 44.49 33.44) (end 44.49 34.43) (width 0.2) (layer "F.Cu") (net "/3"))
 (segment (start 41.8 49.49) (end 28.14 49.49) (width 0.2) (layer "F.Cu") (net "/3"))
 (segment (start 44.49 35.13) (end 44.49 36.02) (width 0.2) (layer "F.Cu") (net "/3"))
 (segment (start 26.11 37.74) (end 26.11 37.76) (width 0.2) (layer "F.Cu") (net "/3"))
 (segment (start 44.49 43.52) (end 44.49 43.51) (width 0.2) (layer "F.Cu") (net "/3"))
 (segment (start 44.39 34.33) (end 26.11 34.33) (width 0.2) (layer "F.Cu") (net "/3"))
 (segment (start 42.01 48.97) (end 42.01 49.28) (width 0.2) (layer "F.Cu") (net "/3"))
 (segment (start 26.15 47.22) (end 26.14 47.23) (width 0.2) (layer "F.Cu") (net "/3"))
 (segment (start 44.49 48.97) (end 42.01 48.97) (width 0.2) (layer "F.Cu") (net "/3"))
 (segment (start 44.49 39.4) (end 44.48 39.39) (width 0.2) (layer "F.Cu") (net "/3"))
 (segment (start 44.49 43.52) (end 44.49 44.4) (width 0.2) (layer "F.Cu") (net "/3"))
 (segment (start 44.49 42.36) (end 44.49 43.52) (width 0.2) (layer "F.Cu") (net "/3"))
 (segment (start 44.49 33.44) (end 26.11 33.44) (width 0.2) (layer "F.Cu") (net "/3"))
 (segment (start 44.1 27.62) (end 44.49 28.01) (width 0.2) (layer "F.Cu") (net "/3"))
 (segment (start 44.49 34.43) (end 44.39 34.33) (width 0.2) (layer "F.Cu") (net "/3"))
 (segment (start 44.49 35.13) (end 26.11 35.13) (width 0.2) (layer "F.Cu") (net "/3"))
 (segment (start 44.49 48.06) (end 44.49 48.97) (width 0.2) (layer "F.Cu") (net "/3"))
 (segment (start 44.49 38.58) (end 26.11 38.58) (width 0.2) (layer "F.Cu") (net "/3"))
 (segment (start 44.49 41.23) (end 44.49 42.36) (width 0.2) (layer "F.Cu") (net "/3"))
 (segment (start 44.49 39.4) (end 44.49 40.22) (width 0.2) (layer "F.Cu") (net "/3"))
 (segment (start 44.49 36.02) (end 44.49 36.85) (width 0.2) (layer "F.Cu") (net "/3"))
 (segment (start 44.49 45.42) (end 44.49 46.26) (width 0.2) (layer "F.Cu") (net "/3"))
 (segment (start 26.11 33.44) (end 26.11 33.42) (width 0.2) (layer "F.Cu") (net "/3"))
 (via (at 42.395 27.62) (size 0.6) (drill 0.3) (layers "F.Cu" "B.Cu") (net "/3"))
 (segment (start 42.295 27.52) (end 42.395 27.62) (width 0.2) (layer "B.Cu") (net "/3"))
 (segment (start 41.08 25.59) (end 40.38 25.59) (width 0.2) (layer "B.Cu") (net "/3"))
 (segment (start 40.38 25.59) (end 39.42 26.55) (width 0.2) (layer "B.Cu") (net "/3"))
 (segment (start 40.45 22.43) (end 40.45 25.52) (width 0.2) (layer "B.Cu") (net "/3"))
 (segment (start 39 20.98) (end 40.45 22.43) (width 0.2) (layer "B.Cu") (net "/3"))
 (segment (start 42.295 27.07) (end 42.295 27.52) (width 0.2) (layer "B.Cu") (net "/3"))
 (segment (start 40.45 25.52) (end 40.38 25.59) (width 0.2) (layer "B.Cu") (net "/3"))
 (segment (start 37.46 20.98) (end 39 20.98) (width 0.2) (layer "B.Cu") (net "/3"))
 (segment (start 39.42 26.55) (end 38.9 26.55) (width 0.2) (layer "B.Cu") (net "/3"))
 (segment (start 38.9 26.55) (end 38.555 26.205) (width 0.2) (layer "B.Cu") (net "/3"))
 (segment (start 42.295 26.805) (end 41.08 25.59) (width 0.2) (layer "B.Cu") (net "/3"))
 (segment (start 42.295 27.07) (end 42.295 26.805) (width 0.2) (layer "B.Cu") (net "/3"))
 (segment (start 37.43 25.5) (end 37.43 28.65) (width 0.2) (layer "F.Cu") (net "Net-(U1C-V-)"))
 (segment (start 41.8 24.88) (end 41.54 24.62) (width 0.2) (layer "F.Cu") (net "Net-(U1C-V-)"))
 (segment (start 40.39 24.63) (end 38.3 24.63) (width 0.2) (layer "F.Cu") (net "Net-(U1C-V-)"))
 (segment (start 38.3 24.63) (end 37.43 25.5) (width 0.2) (layer "F.Cu") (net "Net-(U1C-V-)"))
 (segment (start 41.54 24.62) (end 40.4 24.62) (width 0.2) (layer "F.Cu") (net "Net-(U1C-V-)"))
 (segment (start 40.4 24.62) (end 40.39 24.63) (width 0.2) (layer "F.Cu") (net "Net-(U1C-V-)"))
 (via (at 37.43 28.65) (size 0.6) (drill 0.3) (layers "F.Cu" "B.Cu") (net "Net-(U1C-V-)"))
 (via (at 41.8 24.88) (size 0.6) (drill 0.3) (layers "F.Cu" "B.Cu") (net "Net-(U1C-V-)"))
 (segment (start 39.2 28.59) (end 39.2 28.12) (width 0.2) (layer "B.Cu") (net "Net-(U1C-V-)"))
 (segment (start 37.71 29.04) (end 38.75 29.04) (width 0.2) (layer "B.Cu") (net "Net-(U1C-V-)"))
 (segment (start 37.43 28.65) (end 37.43 28.76) (width 0.2) (layer "B.Cu") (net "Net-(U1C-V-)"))
 (segment (start 41.795 24.885) (end 41.8 24.88) (width 0.2) (layer "B.Cu") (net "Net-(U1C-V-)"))
 (segment (start 39.2 28.12) (end 38.555 27.475) (width 0.2) (layer "B.Cu") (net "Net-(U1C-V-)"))
 (segment (start 38.75 29.04) (end 39.2 28.59) (width 0.2) (layer "B.Cu") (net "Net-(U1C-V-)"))
 (segment (start 41.795 25.42) (end 41.795 24.885) (width 0.2) (layer "B.Cu") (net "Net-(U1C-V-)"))
 (segment (start 37.43 28.76) (end 37.71 29.04) (width 0.2) (layer "B.Cu") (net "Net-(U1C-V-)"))
 (segment (start 41.16 22.83) (end 40.93 22.6) (width 0.2) (layer "F.Cu") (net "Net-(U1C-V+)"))
 (segment (start 34.42 23.06) (end 34.18 23.06) (width 0.2) (layer "F.Cu") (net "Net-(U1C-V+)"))
 (segment (start 40.93 22.6) (end 34.88 22.6) (width 0.2) (layer "F.Cu") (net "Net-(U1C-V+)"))
 (segment (start 34.88 22.6) (end 34.42 23.06) (width 0.2) (layer "F.Cu") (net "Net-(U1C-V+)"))
 (via (at 41.16 22.83) (size 0.6) (drill 0.3) (layers "F.Cu" "B.Cu") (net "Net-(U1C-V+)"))
 (via (at 34.18 23.06) (size 0.6) (drill 0.3) (layers "F.Cu" "B.Cu") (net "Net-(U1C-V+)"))
 (segment (start 42.295 23.77) (end 42.295 23.53759) (width 0.2) (layer "B.Cu") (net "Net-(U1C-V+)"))
 (segment (start 33.605 23.295) (end 33.605 23.665) (width 0.2) (layer "B.Cu") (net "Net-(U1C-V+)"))
 (segment (start 34.18 23.06) (end 33.84 23.06) (width 0.2) (layer "B.Cu") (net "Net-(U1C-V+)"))
 (segment (start 42.295 23.53759) (end 41.58741 22.83) (width 0.2) (layer "B.Cu") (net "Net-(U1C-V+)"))
 (segment (start 33.84 23.06) (end 33.605 23.295) (width 0.2) (layer "B.Cu") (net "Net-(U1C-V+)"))
 (segment (start 41.58741 22.83) (end 41.16 22.83) (width 0.2) (layer "B.Cu") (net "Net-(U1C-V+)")))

